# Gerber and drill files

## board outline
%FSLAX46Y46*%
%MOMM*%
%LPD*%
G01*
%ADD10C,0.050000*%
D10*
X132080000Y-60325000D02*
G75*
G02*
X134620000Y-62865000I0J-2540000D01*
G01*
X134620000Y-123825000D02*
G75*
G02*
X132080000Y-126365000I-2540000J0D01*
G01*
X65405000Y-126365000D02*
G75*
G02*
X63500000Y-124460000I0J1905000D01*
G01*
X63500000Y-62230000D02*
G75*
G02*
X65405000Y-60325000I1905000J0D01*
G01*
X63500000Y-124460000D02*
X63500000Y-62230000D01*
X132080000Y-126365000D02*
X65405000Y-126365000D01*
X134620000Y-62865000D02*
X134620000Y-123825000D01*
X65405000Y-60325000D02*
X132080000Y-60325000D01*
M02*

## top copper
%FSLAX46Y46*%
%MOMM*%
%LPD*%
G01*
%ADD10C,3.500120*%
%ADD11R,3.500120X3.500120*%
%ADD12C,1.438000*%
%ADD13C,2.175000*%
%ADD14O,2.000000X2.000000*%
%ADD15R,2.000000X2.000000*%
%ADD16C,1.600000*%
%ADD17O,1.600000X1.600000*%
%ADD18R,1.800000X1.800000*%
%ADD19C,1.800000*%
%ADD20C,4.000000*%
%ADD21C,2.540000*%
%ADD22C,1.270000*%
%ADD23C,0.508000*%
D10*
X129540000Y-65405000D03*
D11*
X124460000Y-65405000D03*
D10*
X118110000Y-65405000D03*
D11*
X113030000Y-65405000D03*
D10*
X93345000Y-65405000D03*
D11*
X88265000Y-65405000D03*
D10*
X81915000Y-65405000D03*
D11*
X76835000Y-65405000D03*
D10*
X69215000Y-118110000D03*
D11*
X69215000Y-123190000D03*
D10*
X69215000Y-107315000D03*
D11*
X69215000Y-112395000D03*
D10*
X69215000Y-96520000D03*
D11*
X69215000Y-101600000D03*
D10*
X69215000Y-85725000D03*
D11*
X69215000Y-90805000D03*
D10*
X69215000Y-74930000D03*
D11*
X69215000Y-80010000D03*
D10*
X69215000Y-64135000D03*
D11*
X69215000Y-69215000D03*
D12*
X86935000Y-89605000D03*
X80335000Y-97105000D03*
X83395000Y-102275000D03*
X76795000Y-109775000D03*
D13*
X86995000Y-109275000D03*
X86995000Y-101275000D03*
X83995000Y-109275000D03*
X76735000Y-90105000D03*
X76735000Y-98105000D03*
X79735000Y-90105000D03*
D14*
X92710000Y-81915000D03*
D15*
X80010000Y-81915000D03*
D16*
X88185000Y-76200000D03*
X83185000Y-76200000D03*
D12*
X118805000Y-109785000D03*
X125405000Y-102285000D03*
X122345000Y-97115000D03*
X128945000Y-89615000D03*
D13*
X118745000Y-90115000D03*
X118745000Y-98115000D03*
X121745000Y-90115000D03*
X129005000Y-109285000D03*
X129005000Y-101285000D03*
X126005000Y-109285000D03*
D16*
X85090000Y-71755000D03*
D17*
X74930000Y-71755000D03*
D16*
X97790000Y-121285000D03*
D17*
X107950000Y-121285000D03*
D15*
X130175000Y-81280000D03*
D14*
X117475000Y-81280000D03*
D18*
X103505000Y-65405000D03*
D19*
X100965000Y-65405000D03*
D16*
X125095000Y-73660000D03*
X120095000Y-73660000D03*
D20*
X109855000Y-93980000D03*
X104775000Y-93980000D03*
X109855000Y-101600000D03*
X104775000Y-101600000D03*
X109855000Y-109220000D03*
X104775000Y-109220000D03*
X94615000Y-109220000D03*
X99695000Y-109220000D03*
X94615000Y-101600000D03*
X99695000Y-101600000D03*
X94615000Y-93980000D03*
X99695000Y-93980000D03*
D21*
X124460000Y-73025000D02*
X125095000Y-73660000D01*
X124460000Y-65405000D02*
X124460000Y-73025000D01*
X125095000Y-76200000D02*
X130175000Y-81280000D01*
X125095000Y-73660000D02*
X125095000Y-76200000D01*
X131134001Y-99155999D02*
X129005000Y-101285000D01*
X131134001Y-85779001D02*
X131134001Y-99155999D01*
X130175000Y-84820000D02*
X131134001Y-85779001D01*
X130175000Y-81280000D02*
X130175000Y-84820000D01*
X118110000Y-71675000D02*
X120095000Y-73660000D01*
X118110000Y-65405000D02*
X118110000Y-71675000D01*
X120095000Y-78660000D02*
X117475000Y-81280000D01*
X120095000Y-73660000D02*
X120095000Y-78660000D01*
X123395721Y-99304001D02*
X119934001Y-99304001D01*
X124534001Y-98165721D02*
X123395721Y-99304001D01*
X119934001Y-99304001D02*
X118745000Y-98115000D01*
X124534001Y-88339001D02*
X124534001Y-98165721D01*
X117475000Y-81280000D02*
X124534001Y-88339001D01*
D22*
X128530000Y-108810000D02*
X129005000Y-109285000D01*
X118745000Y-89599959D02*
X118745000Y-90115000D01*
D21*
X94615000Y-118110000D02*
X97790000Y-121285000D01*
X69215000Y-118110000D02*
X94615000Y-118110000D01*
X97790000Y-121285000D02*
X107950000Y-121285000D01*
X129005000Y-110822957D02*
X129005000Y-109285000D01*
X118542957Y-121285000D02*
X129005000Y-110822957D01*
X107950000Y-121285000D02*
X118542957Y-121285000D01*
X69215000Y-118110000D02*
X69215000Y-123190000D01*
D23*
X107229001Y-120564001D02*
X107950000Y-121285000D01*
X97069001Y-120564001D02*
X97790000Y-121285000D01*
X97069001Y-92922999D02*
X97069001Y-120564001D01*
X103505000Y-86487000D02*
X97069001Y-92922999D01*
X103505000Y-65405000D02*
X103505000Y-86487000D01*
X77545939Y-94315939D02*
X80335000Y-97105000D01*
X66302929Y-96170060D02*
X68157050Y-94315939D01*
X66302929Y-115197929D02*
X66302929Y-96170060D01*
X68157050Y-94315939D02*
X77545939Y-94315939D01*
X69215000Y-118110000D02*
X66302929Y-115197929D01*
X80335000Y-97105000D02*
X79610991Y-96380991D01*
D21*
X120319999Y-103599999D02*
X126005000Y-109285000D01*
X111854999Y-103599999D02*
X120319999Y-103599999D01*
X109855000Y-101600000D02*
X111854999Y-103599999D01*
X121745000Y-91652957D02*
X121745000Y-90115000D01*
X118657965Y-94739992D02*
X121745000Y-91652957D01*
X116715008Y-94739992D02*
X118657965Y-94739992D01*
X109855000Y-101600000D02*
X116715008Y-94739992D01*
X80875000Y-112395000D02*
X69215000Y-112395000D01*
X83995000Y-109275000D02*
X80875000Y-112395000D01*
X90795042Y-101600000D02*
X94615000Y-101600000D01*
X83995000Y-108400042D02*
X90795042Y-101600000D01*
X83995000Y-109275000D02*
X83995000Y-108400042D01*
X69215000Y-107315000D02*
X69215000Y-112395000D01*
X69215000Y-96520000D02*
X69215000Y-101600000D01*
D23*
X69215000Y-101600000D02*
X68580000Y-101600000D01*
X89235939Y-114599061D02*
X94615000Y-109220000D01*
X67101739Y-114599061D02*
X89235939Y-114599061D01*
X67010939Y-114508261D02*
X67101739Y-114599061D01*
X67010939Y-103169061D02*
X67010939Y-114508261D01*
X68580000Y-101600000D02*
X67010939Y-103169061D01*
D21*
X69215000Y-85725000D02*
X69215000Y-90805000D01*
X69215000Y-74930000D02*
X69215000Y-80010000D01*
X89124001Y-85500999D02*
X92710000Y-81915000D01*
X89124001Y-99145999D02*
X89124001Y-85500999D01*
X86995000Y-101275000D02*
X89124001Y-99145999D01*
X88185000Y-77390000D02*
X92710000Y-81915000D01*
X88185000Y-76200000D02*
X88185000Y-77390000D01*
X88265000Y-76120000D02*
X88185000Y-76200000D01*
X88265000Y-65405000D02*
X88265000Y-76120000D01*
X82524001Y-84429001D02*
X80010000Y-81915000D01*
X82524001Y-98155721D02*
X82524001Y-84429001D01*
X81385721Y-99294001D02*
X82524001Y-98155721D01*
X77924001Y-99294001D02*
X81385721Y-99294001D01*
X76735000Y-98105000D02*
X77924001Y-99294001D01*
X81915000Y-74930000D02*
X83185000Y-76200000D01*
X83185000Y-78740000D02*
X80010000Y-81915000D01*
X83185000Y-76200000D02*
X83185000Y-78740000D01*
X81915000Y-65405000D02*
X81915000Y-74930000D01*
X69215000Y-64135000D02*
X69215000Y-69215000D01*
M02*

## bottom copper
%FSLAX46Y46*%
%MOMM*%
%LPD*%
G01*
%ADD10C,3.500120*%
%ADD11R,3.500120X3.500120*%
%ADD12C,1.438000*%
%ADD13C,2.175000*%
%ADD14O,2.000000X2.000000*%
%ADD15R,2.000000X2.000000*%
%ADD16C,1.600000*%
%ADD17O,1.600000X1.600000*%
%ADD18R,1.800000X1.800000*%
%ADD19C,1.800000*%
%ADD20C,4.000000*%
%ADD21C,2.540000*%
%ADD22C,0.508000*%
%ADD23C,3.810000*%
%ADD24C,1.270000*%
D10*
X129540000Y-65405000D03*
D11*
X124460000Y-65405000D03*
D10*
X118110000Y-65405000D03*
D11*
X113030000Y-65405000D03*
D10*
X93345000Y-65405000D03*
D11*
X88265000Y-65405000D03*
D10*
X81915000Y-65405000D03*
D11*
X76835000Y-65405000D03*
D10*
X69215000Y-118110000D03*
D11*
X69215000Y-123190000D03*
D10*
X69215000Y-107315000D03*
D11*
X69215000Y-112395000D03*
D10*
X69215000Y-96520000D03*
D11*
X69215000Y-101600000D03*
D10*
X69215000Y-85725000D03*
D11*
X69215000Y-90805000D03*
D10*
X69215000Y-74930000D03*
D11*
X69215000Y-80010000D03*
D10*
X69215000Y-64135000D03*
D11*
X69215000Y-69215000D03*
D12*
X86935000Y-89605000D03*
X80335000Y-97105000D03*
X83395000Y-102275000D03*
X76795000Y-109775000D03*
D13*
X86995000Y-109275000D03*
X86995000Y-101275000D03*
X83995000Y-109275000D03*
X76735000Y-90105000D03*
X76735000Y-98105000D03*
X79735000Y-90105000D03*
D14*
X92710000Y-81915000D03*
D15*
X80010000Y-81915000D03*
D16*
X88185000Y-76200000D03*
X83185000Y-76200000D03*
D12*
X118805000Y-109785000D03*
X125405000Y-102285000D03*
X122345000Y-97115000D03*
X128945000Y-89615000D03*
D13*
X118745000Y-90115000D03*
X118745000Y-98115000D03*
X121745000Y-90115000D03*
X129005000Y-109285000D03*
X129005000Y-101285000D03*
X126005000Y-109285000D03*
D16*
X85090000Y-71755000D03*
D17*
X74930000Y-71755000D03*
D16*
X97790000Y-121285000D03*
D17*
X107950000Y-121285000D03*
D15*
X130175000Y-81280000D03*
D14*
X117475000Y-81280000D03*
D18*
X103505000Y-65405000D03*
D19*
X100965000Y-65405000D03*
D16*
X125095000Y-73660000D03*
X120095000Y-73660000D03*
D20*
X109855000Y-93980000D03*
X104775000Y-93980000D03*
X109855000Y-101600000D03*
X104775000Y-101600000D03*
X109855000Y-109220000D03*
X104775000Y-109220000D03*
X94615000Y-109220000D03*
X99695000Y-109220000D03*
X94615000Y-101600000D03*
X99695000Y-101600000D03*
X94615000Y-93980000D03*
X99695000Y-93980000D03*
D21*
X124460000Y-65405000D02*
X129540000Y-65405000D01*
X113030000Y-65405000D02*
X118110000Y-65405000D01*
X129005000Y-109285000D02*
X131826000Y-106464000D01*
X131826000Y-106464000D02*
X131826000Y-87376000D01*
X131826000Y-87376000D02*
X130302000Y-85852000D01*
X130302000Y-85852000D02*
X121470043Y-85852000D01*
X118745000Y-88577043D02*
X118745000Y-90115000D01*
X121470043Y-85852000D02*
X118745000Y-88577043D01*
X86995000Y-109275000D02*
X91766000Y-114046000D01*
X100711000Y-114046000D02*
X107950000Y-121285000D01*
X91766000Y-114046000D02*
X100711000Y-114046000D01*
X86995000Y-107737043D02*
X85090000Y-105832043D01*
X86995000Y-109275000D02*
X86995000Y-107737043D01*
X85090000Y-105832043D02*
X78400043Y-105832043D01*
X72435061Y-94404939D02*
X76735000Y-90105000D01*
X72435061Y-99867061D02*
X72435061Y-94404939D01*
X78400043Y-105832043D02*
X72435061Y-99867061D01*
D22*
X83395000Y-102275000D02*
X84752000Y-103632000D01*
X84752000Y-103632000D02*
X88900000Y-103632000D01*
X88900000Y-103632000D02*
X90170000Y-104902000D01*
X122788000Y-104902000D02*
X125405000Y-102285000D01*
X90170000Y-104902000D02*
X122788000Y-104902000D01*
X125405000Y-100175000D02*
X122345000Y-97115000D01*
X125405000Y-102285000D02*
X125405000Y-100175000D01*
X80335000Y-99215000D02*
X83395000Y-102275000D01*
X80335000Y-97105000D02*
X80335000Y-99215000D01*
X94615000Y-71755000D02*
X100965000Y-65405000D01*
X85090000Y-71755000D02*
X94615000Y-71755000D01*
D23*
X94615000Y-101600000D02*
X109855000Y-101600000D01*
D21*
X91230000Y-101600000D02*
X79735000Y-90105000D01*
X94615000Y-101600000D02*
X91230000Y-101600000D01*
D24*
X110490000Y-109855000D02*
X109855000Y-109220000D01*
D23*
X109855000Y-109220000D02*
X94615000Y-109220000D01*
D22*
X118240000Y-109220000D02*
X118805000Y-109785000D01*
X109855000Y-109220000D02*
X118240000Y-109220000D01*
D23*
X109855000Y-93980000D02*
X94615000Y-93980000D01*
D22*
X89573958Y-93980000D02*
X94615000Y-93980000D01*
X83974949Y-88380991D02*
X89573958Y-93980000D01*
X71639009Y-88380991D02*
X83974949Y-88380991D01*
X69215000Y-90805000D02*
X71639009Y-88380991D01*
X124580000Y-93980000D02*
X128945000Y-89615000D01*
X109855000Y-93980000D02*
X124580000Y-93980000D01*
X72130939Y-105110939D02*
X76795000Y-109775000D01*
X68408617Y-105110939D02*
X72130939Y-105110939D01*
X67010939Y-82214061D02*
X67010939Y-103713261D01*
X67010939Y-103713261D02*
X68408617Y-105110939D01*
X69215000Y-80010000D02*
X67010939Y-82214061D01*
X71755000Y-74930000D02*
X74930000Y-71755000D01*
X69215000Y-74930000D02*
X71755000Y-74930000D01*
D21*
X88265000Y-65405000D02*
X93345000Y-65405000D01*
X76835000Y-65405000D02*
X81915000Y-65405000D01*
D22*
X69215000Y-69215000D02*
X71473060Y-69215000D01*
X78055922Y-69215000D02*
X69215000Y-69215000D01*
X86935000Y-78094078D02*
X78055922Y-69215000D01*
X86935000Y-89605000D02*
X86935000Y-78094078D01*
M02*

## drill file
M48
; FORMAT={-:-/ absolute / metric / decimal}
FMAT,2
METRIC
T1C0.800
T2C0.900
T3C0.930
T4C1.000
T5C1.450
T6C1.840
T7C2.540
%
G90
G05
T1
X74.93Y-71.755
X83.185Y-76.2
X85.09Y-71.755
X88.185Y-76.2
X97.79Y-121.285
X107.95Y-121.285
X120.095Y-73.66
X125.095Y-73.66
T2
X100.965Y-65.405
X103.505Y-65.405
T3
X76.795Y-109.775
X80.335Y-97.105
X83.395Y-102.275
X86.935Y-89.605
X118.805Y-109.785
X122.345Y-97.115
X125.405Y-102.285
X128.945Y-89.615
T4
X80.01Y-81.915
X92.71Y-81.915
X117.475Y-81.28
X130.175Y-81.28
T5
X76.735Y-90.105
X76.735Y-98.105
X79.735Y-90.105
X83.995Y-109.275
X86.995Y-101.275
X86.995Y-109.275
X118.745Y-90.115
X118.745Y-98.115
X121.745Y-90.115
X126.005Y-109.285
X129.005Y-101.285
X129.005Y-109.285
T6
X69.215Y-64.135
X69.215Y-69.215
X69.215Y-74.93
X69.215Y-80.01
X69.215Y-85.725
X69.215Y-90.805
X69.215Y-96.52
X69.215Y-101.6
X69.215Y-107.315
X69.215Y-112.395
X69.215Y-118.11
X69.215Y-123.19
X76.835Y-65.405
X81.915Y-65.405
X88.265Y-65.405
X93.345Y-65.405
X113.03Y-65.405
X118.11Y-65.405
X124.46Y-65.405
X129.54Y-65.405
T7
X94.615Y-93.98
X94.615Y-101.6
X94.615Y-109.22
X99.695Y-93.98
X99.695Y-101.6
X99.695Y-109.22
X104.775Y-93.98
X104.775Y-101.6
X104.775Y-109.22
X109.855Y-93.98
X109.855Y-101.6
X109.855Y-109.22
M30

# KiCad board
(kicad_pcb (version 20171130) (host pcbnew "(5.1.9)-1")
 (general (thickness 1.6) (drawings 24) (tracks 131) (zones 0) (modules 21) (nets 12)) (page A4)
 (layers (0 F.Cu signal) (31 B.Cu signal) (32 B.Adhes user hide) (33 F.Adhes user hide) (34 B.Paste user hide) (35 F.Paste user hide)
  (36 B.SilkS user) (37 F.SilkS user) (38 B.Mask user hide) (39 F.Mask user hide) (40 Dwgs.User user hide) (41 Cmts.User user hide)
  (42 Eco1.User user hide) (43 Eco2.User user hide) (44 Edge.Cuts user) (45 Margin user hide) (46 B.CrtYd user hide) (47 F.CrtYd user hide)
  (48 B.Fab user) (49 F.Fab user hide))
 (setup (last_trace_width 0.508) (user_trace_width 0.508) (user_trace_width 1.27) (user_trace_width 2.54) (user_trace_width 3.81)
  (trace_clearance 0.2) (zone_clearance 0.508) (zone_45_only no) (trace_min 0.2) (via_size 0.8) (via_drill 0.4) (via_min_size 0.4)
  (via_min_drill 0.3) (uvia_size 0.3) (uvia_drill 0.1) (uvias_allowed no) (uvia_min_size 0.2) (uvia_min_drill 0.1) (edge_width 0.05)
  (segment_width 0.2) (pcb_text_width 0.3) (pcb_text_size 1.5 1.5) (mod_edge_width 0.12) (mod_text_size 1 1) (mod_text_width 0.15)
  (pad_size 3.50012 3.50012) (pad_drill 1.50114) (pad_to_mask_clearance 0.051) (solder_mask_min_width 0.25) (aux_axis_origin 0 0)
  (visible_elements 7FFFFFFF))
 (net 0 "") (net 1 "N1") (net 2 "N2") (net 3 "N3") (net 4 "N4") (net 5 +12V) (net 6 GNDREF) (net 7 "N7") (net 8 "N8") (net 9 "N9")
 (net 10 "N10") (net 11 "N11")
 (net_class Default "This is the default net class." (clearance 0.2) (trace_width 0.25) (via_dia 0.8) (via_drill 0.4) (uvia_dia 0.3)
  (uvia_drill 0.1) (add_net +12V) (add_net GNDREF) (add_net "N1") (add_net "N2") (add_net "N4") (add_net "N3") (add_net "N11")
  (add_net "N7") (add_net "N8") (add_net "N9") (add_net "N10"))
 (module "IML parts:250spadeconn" (layer F.Cu) (at 124.46 65.405)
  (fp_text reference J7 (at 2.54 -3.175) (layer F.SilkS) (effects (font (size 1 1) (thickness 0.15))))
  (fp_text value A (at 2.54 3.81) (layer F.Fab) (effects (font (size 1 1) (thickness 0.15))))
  (pad 1 thru_hole circle (at 5.08 0) (size 3.50012 3.50012) (drill 1.84) (layers *.Cu *.Mask) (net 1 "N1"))
  (pad 1 thru_hole rect (at 0 0) (size 3.50012 3.50012) (drill 1.84) (layers *.Cu *.Mask) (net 1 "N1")))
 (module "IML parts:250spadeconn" (layer F.Cu) (at 113.03 65.405)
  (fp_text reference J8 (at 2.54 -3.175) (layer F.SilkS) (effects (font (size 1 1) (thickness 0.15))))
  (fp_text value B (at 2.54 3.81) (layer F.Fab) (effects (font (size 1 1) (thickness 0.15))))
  (pad 1 thru_hole circle (at 5.08 0) (size 3.50012 3.50012) (drill 1.84) (layers *.Cu *.Mask) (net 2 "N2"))
  (pad 1 thru_hole rect (at 0 0) (size 3.50012 3.50012) (drill 1.84) (layers *.Cu *.Mask) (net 2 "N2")))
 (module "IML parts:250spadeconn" (layer F.Cu) (at 88.265 65.405)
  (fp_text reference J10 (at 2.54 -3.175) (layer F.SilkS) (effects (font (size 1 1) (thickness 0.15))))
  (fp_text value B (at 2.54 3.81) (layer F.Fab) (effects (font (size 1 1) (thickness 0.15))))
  (pad 1 thru_hole circle (at 5.08 0) (size 3.50012 3.50012) (drill 1.84) (layers *.Cu *.Mask) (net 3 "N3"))
  (pad 1 thru_hole rect (at 0 0) (size 3.50012 3.50012) (drill 1.84) (layers *.Cu *.Mask) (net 3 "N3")))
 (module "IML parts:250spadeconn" (layer F.Cu) (at 76.835 65.405)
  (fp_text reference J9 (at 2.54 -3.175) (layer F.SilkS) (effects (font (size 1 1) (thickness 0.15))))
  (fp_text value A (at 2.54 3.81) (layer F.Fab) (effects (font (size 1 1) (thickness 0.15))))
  (pad 1 thru_hole circle (at 5.08 0) (size 3.50012 3.50012) (drill 1.84) (layers *.Cu *.Mask) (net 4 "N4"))
  (pad 1 thru_hole rect (at 0 0) (size 3.50012 3.50012) (drill 1.84) (layers *.Cu *.Mask) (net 4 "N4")))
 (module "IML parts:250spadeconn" (layer F.Cu) (at 69.215 123.19 90)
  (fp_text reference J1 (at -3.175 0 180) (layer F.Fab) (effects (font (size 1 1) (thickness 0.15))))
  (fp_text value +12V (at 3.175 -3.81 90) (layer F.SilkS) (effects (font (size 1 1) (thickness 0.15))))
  (pad 1 thru_hole circle (at 5.08 0 90) (size 3.50012 3.50012) (drill 1.84) (layers *.Cu *.Mask) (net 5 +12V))
  (pad 1 thru_hole rect (at 0 0 90) (size 3.50012 3.50012) (drill 1.84) (layers *.Cu *.Mask) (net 5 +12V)))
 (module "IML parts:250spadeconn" (layer F.Cu) (at 69.215 112.395 90)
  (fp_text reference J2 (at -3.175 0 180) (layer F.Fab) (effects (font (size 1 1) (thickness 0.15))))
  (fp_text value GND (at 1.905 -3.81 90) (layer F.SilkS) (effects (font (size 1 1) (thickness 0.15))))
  (pad 1 thru_hole circle (at 5.08 0 90) (size 3.50012 3.50012) (drill 1.84) (layers *.Cu *.Mask) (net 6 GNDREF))
  (pad 1 thru_hole rect (at 0 0 90) (size 3.50012 3.50012) (drill 1.84) (layers *.Cu *.Mask) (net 6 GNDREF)))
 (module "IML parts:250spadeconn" (layer F.Cu) (at 69.215 101.6 90)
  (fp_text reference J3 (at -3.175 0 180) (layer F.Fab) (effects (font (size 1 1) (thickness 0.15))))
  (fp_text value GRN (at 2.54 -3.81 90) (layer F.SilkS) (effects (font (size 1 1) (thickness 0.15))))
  (pad 1 thru_hole circle (at 5.08 0 90) (size 3.50012 3.50012) (drill 1.84) (layers *.Cu *.Mask) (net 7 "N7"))
  (pad 1 thru_hole rect (at 0 0 90) (size 3.50012 3.50012) (drill 1.84) (layers *.Cu *.Mask) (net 7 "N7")))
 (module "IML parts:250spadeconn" (layer F.Cu) (at 69.215 90.805 90)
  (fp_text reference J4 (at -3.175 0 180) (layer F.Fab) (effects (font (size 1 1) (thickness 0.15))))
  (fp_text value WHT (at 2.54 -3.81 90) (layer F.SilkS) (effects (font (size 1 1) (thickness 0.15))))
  (pad 1 thru_hole circle (at 5.08 0 90) (size 3.50012 3.50012) (drill 1.84) (layers *.Cu *.Mask) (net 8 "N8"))
  (pad 1 thru_hole rect (at 0 0 90) (size 3.50012 3.50012) (drill 1.84) (layers *.Cu *.Mask) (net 8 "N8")))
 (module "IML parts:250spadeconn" (layer F.Cu) (at 69.215 80.01 90)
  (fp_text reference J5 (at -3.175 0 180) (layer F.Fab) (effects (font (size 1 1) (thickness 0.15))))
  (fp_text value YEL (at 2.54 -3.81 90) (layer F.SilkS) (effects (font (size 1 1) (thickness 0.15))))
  (pad 1 thru_hole circle (at 5.08 0 90) (size 3.50012 3.50012) (drill 1.84) (layers *.Cu *.Mask) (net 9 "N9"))
  (pad 1 thru_hole rect (at 0 0 90) (size 3.50012 3.50012) (drill 1.84) (layers *.Cu *.Mask) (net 9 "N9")))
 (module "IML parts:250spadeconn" (layer F.Cu) (at 69.215 69.215 90)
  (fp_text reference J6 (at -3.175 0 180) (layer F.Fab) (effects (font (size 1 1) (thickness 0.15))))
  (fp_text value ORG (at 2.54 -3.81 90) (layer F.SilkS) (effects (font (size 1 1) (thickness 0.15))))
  (pad 1 thru_hole circle (at 5.08 0 90) (size 3.50012 3.50012) (drill 1.84) (layers *.Cu *.Mask) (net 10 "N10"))
  (pad 1 thru_hole rect (at 0 0 90) (size 3.50012 3.50012) (drill 1.84) (layers *.Cu *.Mask) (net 10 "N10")))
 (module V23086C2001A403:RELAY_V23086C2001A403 (layer F.Cu) (at 81.915 99.695 270)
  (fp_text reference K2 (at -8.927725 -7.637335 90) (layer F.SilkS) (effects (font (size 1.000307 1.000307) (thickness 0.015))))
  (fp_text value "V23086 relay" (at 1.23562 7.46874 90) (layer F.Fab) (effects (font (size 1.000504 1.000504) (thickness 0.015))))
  (pad 22 thru_hole circle (at -10.09 -5.02 270) (size 1.438 1.438) (drill 0.93) (layers *.Cu *.Mask) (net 10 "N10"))
  (pad 21 thru_hole circle (at -2.59 1.58 270) (size 1.438 1.438) (drill 0.93) (layers *.Cu *.Mask) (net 5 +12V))
  (pad 11 thru_hole circle (at 2.58 -1.48 270) (size 1.438 1.438) (drill 0.93) (layers *.Cu *.Mask) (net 5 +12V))
  (pad 12 thru_hole circle (at 10.08 5.12 270) (size 1.438 1.438) (drill 0.93) (layers *.Cu *.Mask) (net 9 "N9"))
  (pad 13 thru_hole circle (at 9.58 -5.08 270) (size 2.175 2.175) (drill 1.45) (layers *.Cu *.Mask) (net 5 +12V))
  (pad 14 thru_hole circle (at 1.58 -5.08 270) (size 2.175 2.175) (drill 1.45) (layers *.Cu *.Mask) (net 3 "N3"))
  (pad 15 thru_hole circle (at 9.58 -2.08 270) (size 2.175 2.175) (drill 1.45) (layers *.Cu *.Mask) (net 6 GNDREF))
  (pad 23 thru_hole circle (at -9.59 5.18 270) (size 2.175 2.175) (drill 1.45) (layers *.Cu *.Mask) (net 5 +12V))
  (pad 24 thru_hole circle (at -1.59 5.18 270) (size 2.175 2.175) (drill 1.45) (layers *.Cu *.Mask) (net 4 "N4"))
  (pad 25 thru_hole circle (at -9.59 2.18 270) (size 2.175 2.175) (drill 1.45) (layers *.Cu *.Mask) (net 6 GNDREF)))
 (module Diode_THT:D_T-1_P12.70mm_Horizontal (layer F.Cu) (at 80.01 81.915)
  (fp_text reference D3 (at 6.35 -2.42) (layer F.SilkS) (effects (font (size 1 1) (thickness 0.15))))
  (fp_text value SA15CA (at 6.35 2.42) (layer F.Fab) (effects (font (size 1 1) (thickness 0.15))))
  (pad 2 thru_hole oval (at 12.7 0) (size 2 2) (drill 1) (layers *.Cu *.Mask) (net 3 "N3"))
  (pad 1 thru_hole rect (at 0 0) (size 2 2) (drill 1) (layers *.Cu *.Mask) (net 4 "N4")))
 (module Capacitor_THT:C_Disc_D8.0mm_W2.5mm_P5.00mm (layer F.Cu) (at 83.185 76.2)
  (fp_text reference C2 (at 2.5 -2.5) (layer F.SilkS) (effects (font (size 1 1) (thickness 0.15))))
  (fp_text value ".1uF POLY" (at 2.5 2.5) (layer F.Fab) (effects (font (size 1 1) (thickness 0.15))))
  (pad 2 thru_hole circle (at 5 0) (size 1.6 1.6) (drill 0.8) (layers *.Cu *.Mask) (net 3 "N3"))
  (pad 1 thru_hole circle (at 0 0) (size 1.6 1.6) (drill 0.8) (layers *.Cu *.Mask) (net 4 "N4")))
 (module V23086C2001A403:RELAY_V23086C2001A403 (layer F.Cu) (at 123.825 99.695 90)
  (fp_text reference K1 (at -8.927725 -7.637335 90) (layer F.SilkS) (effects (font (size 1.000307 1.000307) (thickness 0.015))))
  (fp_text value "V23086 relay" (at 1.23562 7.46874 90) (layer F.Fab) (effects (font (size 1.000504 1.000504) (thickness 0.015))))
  (pad 22 thru_hole circle (at -10.09 -5.02 90) (size 1.438 1.438) (drill 0.93) (layers *.Cu *.Mask) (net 7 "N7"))
  (pad 21 thru_hole circle (at -2.59 1.58 90) (size 1.438 1.438) (drill 0.93) (layers *.Cu *.Mask) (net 5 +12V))
  (pad 11 thru_hole circle (at 2.58 -1.48 90) (size 1.438 1.438) (drill 0.93) (layers *.Cu *.Mask) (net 5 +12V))
  (pad 12 thru_hole circle (at 10.08 5.12 90) (size 1.438 1.438) (drill 0.93) (layers *.Cu *.Mask) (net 8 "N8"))
  (pad 13 thru_hole circle (at 9.58 -5.08 90) (size 2.175 2.175) (drill 1.45) (layers *.Cu *.Mask) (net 5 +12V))
  (pad 14 thru_hole circle (at 1.58 -5.08 90) (size 2.175 2.175) (drill 1.45) (layers *.Cu *.Mask) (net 2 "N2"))
  (pad 15 thru_hole circle (at 9.58 -2.08 90) (size 2.175 2.175) (drill 1.45) (layers *.Cu *.Mask) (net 6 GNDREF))
  (pad 23 thru_hole circle (at -9.59 5.18 90) (size 2.175 2.175) (drill 1.45) (layers *.Cu *.Mask) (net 5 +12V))
  (pad 24 thru_hole circle (at -1.59 5.18 90) (size 2.175 2.175) (drill 1.45) (layers *.Cu *.Mask) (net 1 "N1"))
  (pad 25 thru_hole circle (at -9.59 2.18 90) (size 2.175 2.175) (drill 1.45) (layers *.Cu *.Mask) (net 6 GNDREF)))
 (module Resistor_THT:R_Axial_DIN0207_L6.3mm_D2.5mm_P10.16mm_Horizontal (layer F.Cu) (at 85.09 71.755 180)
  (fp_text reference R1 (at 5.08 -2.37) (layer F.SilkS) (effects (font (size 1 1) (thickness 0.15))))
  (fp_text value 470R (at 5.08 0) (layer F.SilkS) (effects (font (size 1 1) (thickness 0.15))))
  (pad 1 thru_hole circle (at 0 0 180) (size 1.6 1.6) (drill 0.8) (layers *.Cu *.Mask) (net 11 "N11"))
  (pad 2 thru_hole oval (at 10.16 0 180) (size 1.6 1.6) (drill 0.8) (layers *.Cu *.Mask) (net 9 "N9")))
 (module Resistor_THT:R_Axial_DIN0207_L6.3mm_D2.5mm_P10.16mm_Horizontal (layer F.Cu) (at 97.79 121.285)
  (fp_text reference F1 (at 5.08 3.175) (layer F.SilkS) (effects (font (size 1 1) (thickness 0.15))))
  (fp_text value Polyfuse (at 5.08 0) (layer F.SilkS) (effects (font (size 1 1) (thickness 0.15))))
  (pad 1 thru_hole circle (at 0 0) (size 1.6 1.6) (drill 0.8) (layers *.Cu *.Mask) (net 5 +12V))
  (pad 2 thru_hole oval (at 10.16 0) (size 1.6 1.6) (drill 0.8) (layers *.Cu *.Mask) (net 5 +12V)))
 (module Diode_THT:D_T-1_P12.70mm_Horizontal (layer F.Cu) (at 130.175 81.28 180)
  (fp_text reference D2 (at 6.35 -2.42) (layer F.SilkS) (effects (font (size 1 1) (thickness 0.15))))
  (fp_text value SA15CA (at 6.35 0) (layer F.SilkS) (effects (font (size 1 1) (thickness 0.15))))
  (pad 1 thru_hole rect (at 0 0 180) (size 2 2) (drill 1) (layers *.Cu *.Mask) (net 1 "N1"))
  (pad 2 thru_hole oval (at 12.7 0 180) (size 2 2) (drill 1) (layers *.Cu *.Mask) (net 2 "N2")))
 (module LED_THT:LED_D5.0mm (layer F.Cu) (at 103.505 65.405 180)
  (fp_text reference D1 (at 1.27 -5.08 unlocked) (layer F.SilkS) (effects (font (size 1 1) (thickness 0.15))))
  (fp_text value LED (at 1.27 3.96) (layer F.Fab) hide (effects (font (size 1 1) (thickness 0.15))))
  (pad 1 thru_hole rect (at 0 0 180) (size 1.8 1.8) (drill 0.9) (layers *.Cu *.Mask) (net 5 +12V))
  (pad 2 thru_hole circle (at 2.54 0 180) (size 1.8 1.8) (drill 0.9) (layers *.Cu *.Mask) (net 11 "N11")))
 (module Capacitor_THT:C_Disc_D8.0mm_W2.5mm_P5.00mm (layer F.Cu) (at 125.095 73.66 180)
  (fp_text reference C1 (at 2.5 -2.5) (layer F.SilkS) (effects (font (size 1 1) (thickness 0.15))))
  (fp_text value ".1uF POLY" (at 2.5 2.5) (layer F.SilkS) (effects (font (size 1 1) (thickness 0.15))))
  (pad 1 thru_hole circle (at 0 0 180) (size 1.6 1.6) (drill 0.8) (layers *.Cu *.Mask) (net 1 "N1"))
  (pad 2 thru_hole circle (at 5 0 180) (size 1.6 1.6) (drill 0.8) (layers *.Cu *.Mask) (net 2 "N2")))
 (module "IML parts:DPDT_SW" (layer F.Cu) (at 107.315 101.6 90)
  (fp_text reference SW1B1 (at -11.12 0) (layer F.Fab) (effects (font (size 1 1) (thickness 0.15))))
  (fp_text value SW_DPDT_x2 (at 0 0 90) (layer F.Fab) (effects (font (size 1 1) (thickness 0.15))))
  (pad 3 thru_hole circle (at 7.62 2.54 90) (size 4 4) (drill 2.54) (layers *.Cu *.Mask) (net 8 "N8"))
  (pad 3 thru_hole circle (at 7.62 -2.54 90) (size 4 4) (drill 2.54) (layers *.Cu *.Mask) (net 8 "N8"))
  (pad 2 thru_hole circle (at 0 2.54 90) (size 4 4) (drill 2.54) (layers *.Cu *.Mask) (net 6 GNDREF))
  (pad 2 thru_hole circle (at 0 -2.54 90) (size 4 4) (drill 2.54) (layers *.Cu *.Mask) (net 6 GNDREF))
  (pad 1 thru_hole circle (at -7.62 2.54 90) (size 4 4) (drill 2.54) (layers *.Cu *.Mask) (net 7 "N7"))
  (pad 1 thru_hole circle (at -7.62 -2.54 90) (size 4 4) (drill 2.54) (layers *.Cu *.Mask) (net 7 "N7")))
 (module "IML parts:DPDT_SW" (layer F.Cu) (at 97.155 101.6 90)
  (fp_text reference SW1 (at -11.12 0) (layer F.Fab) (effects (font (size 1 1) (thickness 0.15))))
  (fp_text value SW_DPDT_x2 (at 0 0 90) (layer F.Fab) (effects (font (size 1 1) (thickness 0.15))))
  (pad 1 thru_hole circle (at -7.62 -2.54 90) (size 4 4) (drill 2.54) (layers *.Cu *.Mask) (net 7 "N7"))
  (pad 1 thru_hole circle (at -7.62 2.54 90) (size 4 4) (drill 2.54) (layers *.Cu *.Mask) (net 7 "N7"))
  (pad 2 thru_hole circle (at 0 -2.54 90) (size 4 4) (drill 2.54) (layers *.Cu *.Mask) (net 6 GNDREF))
  (pad 2 thru_hole circle (at 0 2.54 90) (size 4 4) (drill 2.54) (layers *.Cu *.Mask) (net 6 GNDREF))
  (pad 3 thru_hole circle (at 7.62 -2.54 90) (size 4 4) (drill 2.54) (layers *.Cu *.Mask) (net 8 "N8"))
  (pad 3 thru_hole circle (at 7.62 2.54 90) (size 4 4) (drill 2.54) (layers *.Cu *.Mask) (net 8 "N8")))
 (gr_arc (start 132.08 62.865) (end 134.62 62.865) (angle -90) (layer Edge.Cuts) (width 0.05))
 (gr_arc (start 132.08 123.825) (end 132.08 126.365) (angle -90) (layer Edge.Cuts) (width 0.05))
 (gr_arc (start 65.405 124.46) (end 63.5 124.46) (angle -90) (layer Edge.Cuts) (width 0.05))
 (gr_arc (start 65.405 62.23) (end 65.405 60.325) (angle -90) (layer Edge.Cuts) (width 0.05))
 (gr_line (start 63.5 124.46) (end 63.5 62.23) (layer Edge.Cuts) (width 0.05))
 (gr_line (start 132.08 126.365) (end 65.405 126.365) (layer Edge.Cuts) (width 0.05))
 (gr_line (start 134.62 62.865) (end 134.62 123.825) (layer Edge.Cuts) (width 0.05))
 (gr_line (start 65.405 60.325) (end 132.08 60.325) (layer Edge.Cuts) (width 0.05))
 (segment (start 124.46 73.025) (end 125.095 73.66) (width 2.54) (layer F.Cu) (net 1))
 (segment (start 124.46 65.405) (end 124.46 73.025) (width 2.54) (layer F.Cu) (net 1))
 (segment (start 125.095 76.2) (end 130.175 81.28) (width 2.54) (layer F.Cu) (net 1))
 (segment (start 125.095 73.66) (end 125.095 76.2) (width 2.54) (layer F.Cu) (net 1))
 (segment (start 131.134001 99.155999) (end 129.005 101.285) (width 2.54) (layer F.Cu) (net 1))
 (segment (start 131.134001 85.779001) (end 131.134001 99.155999) (width 2.54) (layer F.Cu) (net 1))
 (segment (start 130.175 84.82) (end 131.134001 85.779001) (width 2.54) (layer F.Cu) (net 1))
 (segment (start 130.175 81.28) (end 130.175 84.82) (width 2.54) (layer F.Cu) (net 1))
 (segment (start 124.46 65.405) (end 129.54 65.405) (width 2.54) (layer B.Cu) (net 1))
 (segment (start 118.11 71.675) (end 120.095 73.66) (width 2.54) (layer F.Cu) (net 2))
 (segment (start 118.11 65.405) (end 118.11 71.675) (width 2.54) (layer F.Cu) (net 2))
 (segment (start 120.095 78.66) (end 117.475 81.28) (width 2.54) (layer F.Cu) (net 2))
 (segment (start 120.095 73.66) (end 120.095 78.66) (width 2.54) (layer F.Cu) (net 2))
 (segment (start 123.395721 99.304001) (end 119.934001 99.304001) (width 2.54) (layer F.Cu) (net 2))
 (segment (start 124.534001 98.165721) (end 123.395721 99.304001) (width 2.54) (layer F.Cu) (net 2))
 (segment (start 119.934001 99.304001) (end 118.745 98.115) (width 2.54) (layer F.Cu) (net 2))
 (segment (start 124.534001 88.339001) (end 124.534001 98.165721) (width 2.54) (layer F.Cu) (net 2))
 (segment (start 117.475 81.28) (end 124.534001 88.339001) (width 2.54) (layer F.Cu) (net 2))
 (segment (start 113.03 65.405) (end 118.11 65.405) (width 2.54) (layer B.Cu) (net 2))
 (segment (start 128.53 108.81) (end 129.005 109.285) (width 1.27) (layer F.Cu) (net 5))
 (segment (start 118.745 89.599959) (end 118.745 90.115) (width 1.27) (layer F.Cu) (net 5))
 (segment (start 94.615 118.11) (end 97.79 121.285) (width 2.54) (layer F.Cu) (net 5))
 (segment (start 69.215 118.11) (end 94.615 118.11) (width 2.54) (layer F.Cu) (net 5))
 (segment (start 97.79 121.285) (end 107.95 121.285) (width 2.54) (layer F.Cu) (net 5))
 (segment (start 129.005 110.822957) (end 129.005 109.285) (width 2.54) (layer F.Cu) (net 5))
 (segment (start 118.542957 121.285) (end 129.005 110.822957) (width 2.54) (layer F.Cu) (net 5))
 (segment (start 107.95 121.285) (end 118.542957 121.285) (width 2.54) (layer F.Cu) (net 5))
 (segment (start 69.215 118.11) (end 69.215 123.19) (width 2.54) (layer F.Cu) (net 5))
 (segment (start 129.005 109.285) (end 131.826 106.464) (width 2.54) (layer B.Cu) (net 5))
 (segment (start 131.826 106.464) (end 131.826 87.376) (width 2.54) (layer B.Cu) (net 5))
 (segment (start 131.826 87.376) (end 130.302 85.852) (width 2.54) (layer B.Cu) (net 5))
 (segment (start 130.302 85.852) (end 121.470043 85.852) (width 2.54) (layer B.Cu) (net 5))
 (segment (start 118.745 88.577043) (end 118.745 90.115) (width 2.54) (layer B.Cu) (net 5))
 (segment (start 121.470043 85.852) (end 118.745 88.577043) (width 2.54) (layer B.Cu) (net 5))
 (segment (start 86.995 109.275) (end 91.766 114.046) (width 2.54) (layer B.Cu) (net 5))
 (segment (start 100.711 114.046) (end 107.95 121.285) (width 2.54) (layer B.Cu) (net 5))
 (segment (start 91.766 114.046) (end 100.711 114.046) (width 2.54) (layer B.Cu) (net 5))
 (segment (start 107.229001 120.564001) (end 107.95 121.285) (width 0.508) (layer F.Cu) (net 5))
 (segment (start 97.069001 120.564001) (end 97.79 121.285) (width 0.508) (layer F.Cu) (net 5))
 (segment (start 97.069001 92.922999) (end 97.069001 120.564001) (width 0.508) (layer F.Cu) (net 5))
 (segment (start 103.505 86.487) (end 97.069001 92.922999) (width 0.508) (layer F.Cu) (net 5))
 (segment (start 103.505 65.405) (end 103.505 86.487) (width 0.508) (layer F.Cu) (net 5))
 (segment (start 77.545939 94.315939) (end 80.335 97.105) (width 0.508) (layer F.Cu) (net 5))
 (segment (start 66.302929 96.17006) (end 68.15705 94.315939) (width 0.508) (layer F.Cu) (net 5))
 (segment (start 66.302929 115.197929) (end 66.302929 96.17006) (width 0.508) (layer F.Cu) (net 5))
 (segment (start 68.15705 94.315939) (end 77.545939 94.315939) (width 0.508) (layer F.Cu) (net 5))
 (segment (start 69.215 118.11) (end 66.302929 115.197929) (width 0.508) (layer F.Cu) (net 5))
 (segment (start 80.335 97.105) (end 79.610991 96.380991) (width 0.508) (layer F.Cu) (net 5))
 (segment (start 86.995 107.737043) (end 85.09 105.832043) (width 2.54) (layer B.Cu) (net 5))
 (segment (start 86.995 109.275) (end 86.995 107.737043) (width 2.54) (layer B.Cu) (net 5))
 (segment (start 85.09 105.832043) (end 78.400043 105.832043) (width 2.54) (layer B.Cu) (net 5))
 (segment (start 72.435061 94.404939) (end 76.735 90.105) (width 2.54) (layer B.Cu) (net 5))
 (segment (start 72.435061 99.867061) (end 72.435061 94.404939) (width 2.54) (layer B.Cu) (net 5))
 (segment (start 78.400043 105.832043) (end 72.435061 99.867061) (width 2.54) (layer B.Cu) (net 5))
 (segment (start 83.395 102.275) (end 84.752 103.632) (width 0.508) (layer B.Cu) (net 5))
 (segment (start 84.752 103.632) (end 88.9 103.632) (width 0.508) (layer B.Cu) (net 5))
 (segment (start 88.9 103.632) (end 90.17 104.902) (width 0.508) (layer B.Cu) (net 5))
 (segment (start 122.788 104.902) (end 125.405 102.285) (width 0.508) (layer B.Cu) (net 5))
 (segment (start 90.17 104.902) (end 122.788 104.902) (width 0.508) (layer B.Cu) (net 5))
 (segment (start 125.405 100.175) (end 122.345 97.115) (width 0.508) (layer B.Cu) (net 5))
 (segment (start 125.405 102.285) (end 125.405 100.175) (width 0.508) (layer B.Cu) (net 5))
 (segment (start 80.335 99.215) (end 83.395 102.275) (width 0.508) (layer B.Cu) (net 5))
 (segment (start 80.335 97.105) (end 80.335 99.215) (width 0.508) (layer B.Cu) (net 5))
 (segment (start 94.615 71.755) (end 100.965 65.405) (width 0.508) (layer B.Cu) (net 11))
 (segment (start 85.09 71.755) (end 94.615 71.755) (width 0.508) (layer B.Cu) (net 11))
 (segment (start 94.615 101.6) (end 109.855 101.6) (width 3.81) (layer B.Cu) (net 6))
 (segment (start 120.319999 103.599999) (end 126.005 109.285) (width 2.54) (layer F.Cu) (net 6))
 (segment (start 111.854999 103.599999) (end 120.319999 103.599999) (width 2.54) (layer F.Cu) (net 6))
 (segment (start 109.855 101.6) (end 111.854999 103.599999) (width 2.54) (layer F.Cu) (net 6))
 (segment (start 121.745 91.652957) (end 121.745 90.115) (width 2.54) (layer F.Cu) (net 6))
 (segment (start 118.657965 94.739992) (end 121.745 91.652957) (width 2.54) (layer F.Cu) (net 6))
 (segment (start 116.715008 94.739992) (end 118.657965 94.739992) (width 2.54) (layer F.Cu) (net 6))
 (segment (start 109.855 101.6) (end 116.715008 94.739992) (width 2.54) (layer F.Cu) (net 6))
 (segment (start 80.875 112.395) (end 69.215 112.395) (width 2.54) (layer F.Cu) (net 6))
 (segment (start 83.995 109.275) (end 80.875 112.395) (width 2.54) (layer F.Cu) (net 6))
 (segment (start 91.23 101.6) (end 79.735 90.105) (width 2.54) (layer B.Cu) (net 6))
 (segment (start 94.615 101.6) (end 91.23 101.6) (width 2.54) (layer B.Cu) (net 6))
 (segment (start 90.795042 101.6) (end 94.615 101.6) (width 2.54) (layer F.Cu) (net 6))
 (segment (start 83.995 108.400042) (end 90.795042 101.6) (width 2.54) (layer F.Cu) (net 6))
 (segment (start 83.995 109.275) (end 83.995 108.400042) (width 2.54) (layer F.Cu) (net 6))
 (segment (start 69.215 107.315) (end 69.215 112.395) (width 2.54) (layer F.Cu) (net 6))
 (segment (start 110.49 109.855) (end 109.855 109.22) (width 1.27) (layer B.Cu) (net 7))
 (segment (start 109.855 109.22) (end 94.615 109.22) (width 3.81) (layer B.Cu) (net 7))
 (segment (start 69.215 96.52) (end 69.215 101.6) (width 2.54) (layer F.Cu) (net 7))
 (segment (start 69.215 101.6) (end 68.58 101.6) (width 0.508) (layer F.Cu) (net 7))
 (segment (start 89.235939 114.599061) (end 94.615 109.22) (width 0.508) (layer F.Cu) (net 7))
 (segment (start 67.101739 114.599061) (end 89.235939 114.599061) (width 0.508) (layer F.Cu) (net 7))
 (segment (start 67.010939 114.508261) (end 67.101739 114.599061) (width 0.508) (layer F.Cu) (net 7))
 (segment (start 67.010939 103.169061) (end 67.010939 114.508261) (width 0.508) (layer F.Cu) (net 7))
 (segment (start 68.58 101.6) (end 67.010939 103.169061) (width 0.508) (layer F.Cu) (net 7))
 (segment (start 118.24 109.22) (end 118.805 109.785) (width 0.508) (layer B.Cu) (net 7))
 (segment (start 109.855 109.22) (end 118.24 109.22) (width 0.508) (layer B.Cu) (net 7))
 (segment (start 109.855 93.98) (end 94.615 93.98) (width 3.81) (layer B.Cu) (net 8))
 (segment (start 89.573958 93.98) (end 94.615 93.98) (width 0.508) (layer B.Cu) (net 8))
 (segment (start 83.974949 88.380991) (end 89.573958 93.98) (width 0.508) (layer B.Cu) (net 8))
 (segment (start 71.639009 88.380991) (end 83.974949 88.380991) (width 0.508) (layer B.Cu) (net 8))
 (segment (start 69.215 90.805) (end 71.639009 88.380991) (width 0.508) (layer B.Cu) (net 8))
 (segment (start 69.215 85.725) (end 69.215 90.805) (width 2.54) (layer F.Cu) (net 8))
 (segment (start 124.58 93.98) (end 128.945 89.615) (width 0.508) (layer B.Cu) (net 8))
 (segment (start 109.855 93.98) (end 124.58 93.98) (width 0.508) (layer B.Cu) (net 8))
 (segment (start 72.130939 105.110939) (end 76.795 109.775) (width 0.508) (layer B.Cu) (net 9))
 (segment (start 68.408617 105.110939) (end 72.130939 105.110939) (width 0.508) (layer B.Cu) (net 9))
 (segment (start 67.010939 82.214061) (end 67.010939 103.713261) (width 0.508) (layer B.Cu) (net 9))
 (segment (start 67.010939 103.713261) (end 68.408617 105.110939) (width 0.508) (layer B.Cu) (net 9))
 (segment (start 69.215 80.01) (end 67.010939 82.214061) (width 0.508) (layer B.Cu) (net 9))
 (segment (start 71.755 74.93) (end 74.93 71.755) (width 0.508) (layer B.Cu) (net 9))
 (segment (start 69.215 74.93) (end 71.755 74.93) (width 0.508) (layer B.Cu) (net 9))
 (segment (start 69.215 74.93) (end 69.215 80.01) (width 2.54) (layer F.Cu) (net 9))
 (segment (start 89.124001 85.500999) (end 92.71 81.915) (width 2.54) (layer F.Cu) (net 3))
 (segment (start 89.124001 99.145999) (end 89.124001 85.500999) (width 2.54) (layer F.Cu) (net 3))
 (segment (start 86.995 101.275) (end 89.124001 99.145999) (width 2.54) (layer F.Cu) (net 3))
 (segment (start 88.185 77.39) (end 92.71 81.915) (width 2.54) (layer F.Cu) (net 3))
 (segment (start 88.185 76.2) (end 88.185 77.39) (width 2.54) (layer F.Cu) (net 3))
 (segment (start 88.265 76.12) (end 88.185 76.2) (width 2.54) (layer F.Cu) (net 3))
 (segment (start 88.265 65.405) (end 88.265 76.12) (width 2.54) (layer F.Cu) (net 3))
 (segment (start 88.265 65.405) (end 93.345 65.405) (width 2.54) (layer B.Cu) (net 3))
 (segment (start 82.524001 84.429001) (end 80.01 81.915) (width 2.54) (layer F.Cu) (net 4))
 (segment (start 82.524001 98.155721) (end 82.524001 84.429001) (width 2.54) (layer F.Cu) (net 4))
 (segment (start 81.385721 99.294001) (end 82.524001 98.155721) (width 2.54) (layer F.Cu) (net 4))
 (segment (start 77.924001 99.294001) (end 81.385721 99.294001) (width 2.54) (layer F.Cu) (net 4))
 (segment (start 76.735 98.105) (end 77.924001 99.294001) (width 2.54) (layer F.Cu) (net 4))
 (segment (start 81.915 74.93) (end 83.185 76.2) (width 2.54) (layer F.Cu) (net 4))
 (segment (start 83.185 78.74) (end 80.01 81.915) (width 2.54) (layer F.Cu) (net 4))
 (segment (start 83.185 76.2) (end 83.185 78.74) (width 2.54) (layer F.Cu) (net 4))
 (segment (start 81.915 65.405) (end 81.915 74.93) (width 2.54) (layer F.Cu) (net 4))
 (segment (start 76.835 65.405) (end 81.915 65.405) (width 2.54) (layer B.Cu) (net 4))
 (segment (start 69.215 69.215) (end 71.47306 69.215) (width 0.508) (layer B.Cu) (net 10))
 (segment (start 78.055922 69.215) (end 69.215 69.215) (width 0.508) (layer B.Cu) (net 10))
 (segment (start 86.935 78.094078) (end 78.055922 69.215) (width 0.508) (layer B.Cu) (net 10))
 (segment (start 86.935 89.605) (end 86.935 78.094078) (width 0.508) (layer B.Cu) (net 10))
 (segment (start 69.215 64.135) (end 69.215 69.215) (width 2.54) (layer F.Cu) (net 10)))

